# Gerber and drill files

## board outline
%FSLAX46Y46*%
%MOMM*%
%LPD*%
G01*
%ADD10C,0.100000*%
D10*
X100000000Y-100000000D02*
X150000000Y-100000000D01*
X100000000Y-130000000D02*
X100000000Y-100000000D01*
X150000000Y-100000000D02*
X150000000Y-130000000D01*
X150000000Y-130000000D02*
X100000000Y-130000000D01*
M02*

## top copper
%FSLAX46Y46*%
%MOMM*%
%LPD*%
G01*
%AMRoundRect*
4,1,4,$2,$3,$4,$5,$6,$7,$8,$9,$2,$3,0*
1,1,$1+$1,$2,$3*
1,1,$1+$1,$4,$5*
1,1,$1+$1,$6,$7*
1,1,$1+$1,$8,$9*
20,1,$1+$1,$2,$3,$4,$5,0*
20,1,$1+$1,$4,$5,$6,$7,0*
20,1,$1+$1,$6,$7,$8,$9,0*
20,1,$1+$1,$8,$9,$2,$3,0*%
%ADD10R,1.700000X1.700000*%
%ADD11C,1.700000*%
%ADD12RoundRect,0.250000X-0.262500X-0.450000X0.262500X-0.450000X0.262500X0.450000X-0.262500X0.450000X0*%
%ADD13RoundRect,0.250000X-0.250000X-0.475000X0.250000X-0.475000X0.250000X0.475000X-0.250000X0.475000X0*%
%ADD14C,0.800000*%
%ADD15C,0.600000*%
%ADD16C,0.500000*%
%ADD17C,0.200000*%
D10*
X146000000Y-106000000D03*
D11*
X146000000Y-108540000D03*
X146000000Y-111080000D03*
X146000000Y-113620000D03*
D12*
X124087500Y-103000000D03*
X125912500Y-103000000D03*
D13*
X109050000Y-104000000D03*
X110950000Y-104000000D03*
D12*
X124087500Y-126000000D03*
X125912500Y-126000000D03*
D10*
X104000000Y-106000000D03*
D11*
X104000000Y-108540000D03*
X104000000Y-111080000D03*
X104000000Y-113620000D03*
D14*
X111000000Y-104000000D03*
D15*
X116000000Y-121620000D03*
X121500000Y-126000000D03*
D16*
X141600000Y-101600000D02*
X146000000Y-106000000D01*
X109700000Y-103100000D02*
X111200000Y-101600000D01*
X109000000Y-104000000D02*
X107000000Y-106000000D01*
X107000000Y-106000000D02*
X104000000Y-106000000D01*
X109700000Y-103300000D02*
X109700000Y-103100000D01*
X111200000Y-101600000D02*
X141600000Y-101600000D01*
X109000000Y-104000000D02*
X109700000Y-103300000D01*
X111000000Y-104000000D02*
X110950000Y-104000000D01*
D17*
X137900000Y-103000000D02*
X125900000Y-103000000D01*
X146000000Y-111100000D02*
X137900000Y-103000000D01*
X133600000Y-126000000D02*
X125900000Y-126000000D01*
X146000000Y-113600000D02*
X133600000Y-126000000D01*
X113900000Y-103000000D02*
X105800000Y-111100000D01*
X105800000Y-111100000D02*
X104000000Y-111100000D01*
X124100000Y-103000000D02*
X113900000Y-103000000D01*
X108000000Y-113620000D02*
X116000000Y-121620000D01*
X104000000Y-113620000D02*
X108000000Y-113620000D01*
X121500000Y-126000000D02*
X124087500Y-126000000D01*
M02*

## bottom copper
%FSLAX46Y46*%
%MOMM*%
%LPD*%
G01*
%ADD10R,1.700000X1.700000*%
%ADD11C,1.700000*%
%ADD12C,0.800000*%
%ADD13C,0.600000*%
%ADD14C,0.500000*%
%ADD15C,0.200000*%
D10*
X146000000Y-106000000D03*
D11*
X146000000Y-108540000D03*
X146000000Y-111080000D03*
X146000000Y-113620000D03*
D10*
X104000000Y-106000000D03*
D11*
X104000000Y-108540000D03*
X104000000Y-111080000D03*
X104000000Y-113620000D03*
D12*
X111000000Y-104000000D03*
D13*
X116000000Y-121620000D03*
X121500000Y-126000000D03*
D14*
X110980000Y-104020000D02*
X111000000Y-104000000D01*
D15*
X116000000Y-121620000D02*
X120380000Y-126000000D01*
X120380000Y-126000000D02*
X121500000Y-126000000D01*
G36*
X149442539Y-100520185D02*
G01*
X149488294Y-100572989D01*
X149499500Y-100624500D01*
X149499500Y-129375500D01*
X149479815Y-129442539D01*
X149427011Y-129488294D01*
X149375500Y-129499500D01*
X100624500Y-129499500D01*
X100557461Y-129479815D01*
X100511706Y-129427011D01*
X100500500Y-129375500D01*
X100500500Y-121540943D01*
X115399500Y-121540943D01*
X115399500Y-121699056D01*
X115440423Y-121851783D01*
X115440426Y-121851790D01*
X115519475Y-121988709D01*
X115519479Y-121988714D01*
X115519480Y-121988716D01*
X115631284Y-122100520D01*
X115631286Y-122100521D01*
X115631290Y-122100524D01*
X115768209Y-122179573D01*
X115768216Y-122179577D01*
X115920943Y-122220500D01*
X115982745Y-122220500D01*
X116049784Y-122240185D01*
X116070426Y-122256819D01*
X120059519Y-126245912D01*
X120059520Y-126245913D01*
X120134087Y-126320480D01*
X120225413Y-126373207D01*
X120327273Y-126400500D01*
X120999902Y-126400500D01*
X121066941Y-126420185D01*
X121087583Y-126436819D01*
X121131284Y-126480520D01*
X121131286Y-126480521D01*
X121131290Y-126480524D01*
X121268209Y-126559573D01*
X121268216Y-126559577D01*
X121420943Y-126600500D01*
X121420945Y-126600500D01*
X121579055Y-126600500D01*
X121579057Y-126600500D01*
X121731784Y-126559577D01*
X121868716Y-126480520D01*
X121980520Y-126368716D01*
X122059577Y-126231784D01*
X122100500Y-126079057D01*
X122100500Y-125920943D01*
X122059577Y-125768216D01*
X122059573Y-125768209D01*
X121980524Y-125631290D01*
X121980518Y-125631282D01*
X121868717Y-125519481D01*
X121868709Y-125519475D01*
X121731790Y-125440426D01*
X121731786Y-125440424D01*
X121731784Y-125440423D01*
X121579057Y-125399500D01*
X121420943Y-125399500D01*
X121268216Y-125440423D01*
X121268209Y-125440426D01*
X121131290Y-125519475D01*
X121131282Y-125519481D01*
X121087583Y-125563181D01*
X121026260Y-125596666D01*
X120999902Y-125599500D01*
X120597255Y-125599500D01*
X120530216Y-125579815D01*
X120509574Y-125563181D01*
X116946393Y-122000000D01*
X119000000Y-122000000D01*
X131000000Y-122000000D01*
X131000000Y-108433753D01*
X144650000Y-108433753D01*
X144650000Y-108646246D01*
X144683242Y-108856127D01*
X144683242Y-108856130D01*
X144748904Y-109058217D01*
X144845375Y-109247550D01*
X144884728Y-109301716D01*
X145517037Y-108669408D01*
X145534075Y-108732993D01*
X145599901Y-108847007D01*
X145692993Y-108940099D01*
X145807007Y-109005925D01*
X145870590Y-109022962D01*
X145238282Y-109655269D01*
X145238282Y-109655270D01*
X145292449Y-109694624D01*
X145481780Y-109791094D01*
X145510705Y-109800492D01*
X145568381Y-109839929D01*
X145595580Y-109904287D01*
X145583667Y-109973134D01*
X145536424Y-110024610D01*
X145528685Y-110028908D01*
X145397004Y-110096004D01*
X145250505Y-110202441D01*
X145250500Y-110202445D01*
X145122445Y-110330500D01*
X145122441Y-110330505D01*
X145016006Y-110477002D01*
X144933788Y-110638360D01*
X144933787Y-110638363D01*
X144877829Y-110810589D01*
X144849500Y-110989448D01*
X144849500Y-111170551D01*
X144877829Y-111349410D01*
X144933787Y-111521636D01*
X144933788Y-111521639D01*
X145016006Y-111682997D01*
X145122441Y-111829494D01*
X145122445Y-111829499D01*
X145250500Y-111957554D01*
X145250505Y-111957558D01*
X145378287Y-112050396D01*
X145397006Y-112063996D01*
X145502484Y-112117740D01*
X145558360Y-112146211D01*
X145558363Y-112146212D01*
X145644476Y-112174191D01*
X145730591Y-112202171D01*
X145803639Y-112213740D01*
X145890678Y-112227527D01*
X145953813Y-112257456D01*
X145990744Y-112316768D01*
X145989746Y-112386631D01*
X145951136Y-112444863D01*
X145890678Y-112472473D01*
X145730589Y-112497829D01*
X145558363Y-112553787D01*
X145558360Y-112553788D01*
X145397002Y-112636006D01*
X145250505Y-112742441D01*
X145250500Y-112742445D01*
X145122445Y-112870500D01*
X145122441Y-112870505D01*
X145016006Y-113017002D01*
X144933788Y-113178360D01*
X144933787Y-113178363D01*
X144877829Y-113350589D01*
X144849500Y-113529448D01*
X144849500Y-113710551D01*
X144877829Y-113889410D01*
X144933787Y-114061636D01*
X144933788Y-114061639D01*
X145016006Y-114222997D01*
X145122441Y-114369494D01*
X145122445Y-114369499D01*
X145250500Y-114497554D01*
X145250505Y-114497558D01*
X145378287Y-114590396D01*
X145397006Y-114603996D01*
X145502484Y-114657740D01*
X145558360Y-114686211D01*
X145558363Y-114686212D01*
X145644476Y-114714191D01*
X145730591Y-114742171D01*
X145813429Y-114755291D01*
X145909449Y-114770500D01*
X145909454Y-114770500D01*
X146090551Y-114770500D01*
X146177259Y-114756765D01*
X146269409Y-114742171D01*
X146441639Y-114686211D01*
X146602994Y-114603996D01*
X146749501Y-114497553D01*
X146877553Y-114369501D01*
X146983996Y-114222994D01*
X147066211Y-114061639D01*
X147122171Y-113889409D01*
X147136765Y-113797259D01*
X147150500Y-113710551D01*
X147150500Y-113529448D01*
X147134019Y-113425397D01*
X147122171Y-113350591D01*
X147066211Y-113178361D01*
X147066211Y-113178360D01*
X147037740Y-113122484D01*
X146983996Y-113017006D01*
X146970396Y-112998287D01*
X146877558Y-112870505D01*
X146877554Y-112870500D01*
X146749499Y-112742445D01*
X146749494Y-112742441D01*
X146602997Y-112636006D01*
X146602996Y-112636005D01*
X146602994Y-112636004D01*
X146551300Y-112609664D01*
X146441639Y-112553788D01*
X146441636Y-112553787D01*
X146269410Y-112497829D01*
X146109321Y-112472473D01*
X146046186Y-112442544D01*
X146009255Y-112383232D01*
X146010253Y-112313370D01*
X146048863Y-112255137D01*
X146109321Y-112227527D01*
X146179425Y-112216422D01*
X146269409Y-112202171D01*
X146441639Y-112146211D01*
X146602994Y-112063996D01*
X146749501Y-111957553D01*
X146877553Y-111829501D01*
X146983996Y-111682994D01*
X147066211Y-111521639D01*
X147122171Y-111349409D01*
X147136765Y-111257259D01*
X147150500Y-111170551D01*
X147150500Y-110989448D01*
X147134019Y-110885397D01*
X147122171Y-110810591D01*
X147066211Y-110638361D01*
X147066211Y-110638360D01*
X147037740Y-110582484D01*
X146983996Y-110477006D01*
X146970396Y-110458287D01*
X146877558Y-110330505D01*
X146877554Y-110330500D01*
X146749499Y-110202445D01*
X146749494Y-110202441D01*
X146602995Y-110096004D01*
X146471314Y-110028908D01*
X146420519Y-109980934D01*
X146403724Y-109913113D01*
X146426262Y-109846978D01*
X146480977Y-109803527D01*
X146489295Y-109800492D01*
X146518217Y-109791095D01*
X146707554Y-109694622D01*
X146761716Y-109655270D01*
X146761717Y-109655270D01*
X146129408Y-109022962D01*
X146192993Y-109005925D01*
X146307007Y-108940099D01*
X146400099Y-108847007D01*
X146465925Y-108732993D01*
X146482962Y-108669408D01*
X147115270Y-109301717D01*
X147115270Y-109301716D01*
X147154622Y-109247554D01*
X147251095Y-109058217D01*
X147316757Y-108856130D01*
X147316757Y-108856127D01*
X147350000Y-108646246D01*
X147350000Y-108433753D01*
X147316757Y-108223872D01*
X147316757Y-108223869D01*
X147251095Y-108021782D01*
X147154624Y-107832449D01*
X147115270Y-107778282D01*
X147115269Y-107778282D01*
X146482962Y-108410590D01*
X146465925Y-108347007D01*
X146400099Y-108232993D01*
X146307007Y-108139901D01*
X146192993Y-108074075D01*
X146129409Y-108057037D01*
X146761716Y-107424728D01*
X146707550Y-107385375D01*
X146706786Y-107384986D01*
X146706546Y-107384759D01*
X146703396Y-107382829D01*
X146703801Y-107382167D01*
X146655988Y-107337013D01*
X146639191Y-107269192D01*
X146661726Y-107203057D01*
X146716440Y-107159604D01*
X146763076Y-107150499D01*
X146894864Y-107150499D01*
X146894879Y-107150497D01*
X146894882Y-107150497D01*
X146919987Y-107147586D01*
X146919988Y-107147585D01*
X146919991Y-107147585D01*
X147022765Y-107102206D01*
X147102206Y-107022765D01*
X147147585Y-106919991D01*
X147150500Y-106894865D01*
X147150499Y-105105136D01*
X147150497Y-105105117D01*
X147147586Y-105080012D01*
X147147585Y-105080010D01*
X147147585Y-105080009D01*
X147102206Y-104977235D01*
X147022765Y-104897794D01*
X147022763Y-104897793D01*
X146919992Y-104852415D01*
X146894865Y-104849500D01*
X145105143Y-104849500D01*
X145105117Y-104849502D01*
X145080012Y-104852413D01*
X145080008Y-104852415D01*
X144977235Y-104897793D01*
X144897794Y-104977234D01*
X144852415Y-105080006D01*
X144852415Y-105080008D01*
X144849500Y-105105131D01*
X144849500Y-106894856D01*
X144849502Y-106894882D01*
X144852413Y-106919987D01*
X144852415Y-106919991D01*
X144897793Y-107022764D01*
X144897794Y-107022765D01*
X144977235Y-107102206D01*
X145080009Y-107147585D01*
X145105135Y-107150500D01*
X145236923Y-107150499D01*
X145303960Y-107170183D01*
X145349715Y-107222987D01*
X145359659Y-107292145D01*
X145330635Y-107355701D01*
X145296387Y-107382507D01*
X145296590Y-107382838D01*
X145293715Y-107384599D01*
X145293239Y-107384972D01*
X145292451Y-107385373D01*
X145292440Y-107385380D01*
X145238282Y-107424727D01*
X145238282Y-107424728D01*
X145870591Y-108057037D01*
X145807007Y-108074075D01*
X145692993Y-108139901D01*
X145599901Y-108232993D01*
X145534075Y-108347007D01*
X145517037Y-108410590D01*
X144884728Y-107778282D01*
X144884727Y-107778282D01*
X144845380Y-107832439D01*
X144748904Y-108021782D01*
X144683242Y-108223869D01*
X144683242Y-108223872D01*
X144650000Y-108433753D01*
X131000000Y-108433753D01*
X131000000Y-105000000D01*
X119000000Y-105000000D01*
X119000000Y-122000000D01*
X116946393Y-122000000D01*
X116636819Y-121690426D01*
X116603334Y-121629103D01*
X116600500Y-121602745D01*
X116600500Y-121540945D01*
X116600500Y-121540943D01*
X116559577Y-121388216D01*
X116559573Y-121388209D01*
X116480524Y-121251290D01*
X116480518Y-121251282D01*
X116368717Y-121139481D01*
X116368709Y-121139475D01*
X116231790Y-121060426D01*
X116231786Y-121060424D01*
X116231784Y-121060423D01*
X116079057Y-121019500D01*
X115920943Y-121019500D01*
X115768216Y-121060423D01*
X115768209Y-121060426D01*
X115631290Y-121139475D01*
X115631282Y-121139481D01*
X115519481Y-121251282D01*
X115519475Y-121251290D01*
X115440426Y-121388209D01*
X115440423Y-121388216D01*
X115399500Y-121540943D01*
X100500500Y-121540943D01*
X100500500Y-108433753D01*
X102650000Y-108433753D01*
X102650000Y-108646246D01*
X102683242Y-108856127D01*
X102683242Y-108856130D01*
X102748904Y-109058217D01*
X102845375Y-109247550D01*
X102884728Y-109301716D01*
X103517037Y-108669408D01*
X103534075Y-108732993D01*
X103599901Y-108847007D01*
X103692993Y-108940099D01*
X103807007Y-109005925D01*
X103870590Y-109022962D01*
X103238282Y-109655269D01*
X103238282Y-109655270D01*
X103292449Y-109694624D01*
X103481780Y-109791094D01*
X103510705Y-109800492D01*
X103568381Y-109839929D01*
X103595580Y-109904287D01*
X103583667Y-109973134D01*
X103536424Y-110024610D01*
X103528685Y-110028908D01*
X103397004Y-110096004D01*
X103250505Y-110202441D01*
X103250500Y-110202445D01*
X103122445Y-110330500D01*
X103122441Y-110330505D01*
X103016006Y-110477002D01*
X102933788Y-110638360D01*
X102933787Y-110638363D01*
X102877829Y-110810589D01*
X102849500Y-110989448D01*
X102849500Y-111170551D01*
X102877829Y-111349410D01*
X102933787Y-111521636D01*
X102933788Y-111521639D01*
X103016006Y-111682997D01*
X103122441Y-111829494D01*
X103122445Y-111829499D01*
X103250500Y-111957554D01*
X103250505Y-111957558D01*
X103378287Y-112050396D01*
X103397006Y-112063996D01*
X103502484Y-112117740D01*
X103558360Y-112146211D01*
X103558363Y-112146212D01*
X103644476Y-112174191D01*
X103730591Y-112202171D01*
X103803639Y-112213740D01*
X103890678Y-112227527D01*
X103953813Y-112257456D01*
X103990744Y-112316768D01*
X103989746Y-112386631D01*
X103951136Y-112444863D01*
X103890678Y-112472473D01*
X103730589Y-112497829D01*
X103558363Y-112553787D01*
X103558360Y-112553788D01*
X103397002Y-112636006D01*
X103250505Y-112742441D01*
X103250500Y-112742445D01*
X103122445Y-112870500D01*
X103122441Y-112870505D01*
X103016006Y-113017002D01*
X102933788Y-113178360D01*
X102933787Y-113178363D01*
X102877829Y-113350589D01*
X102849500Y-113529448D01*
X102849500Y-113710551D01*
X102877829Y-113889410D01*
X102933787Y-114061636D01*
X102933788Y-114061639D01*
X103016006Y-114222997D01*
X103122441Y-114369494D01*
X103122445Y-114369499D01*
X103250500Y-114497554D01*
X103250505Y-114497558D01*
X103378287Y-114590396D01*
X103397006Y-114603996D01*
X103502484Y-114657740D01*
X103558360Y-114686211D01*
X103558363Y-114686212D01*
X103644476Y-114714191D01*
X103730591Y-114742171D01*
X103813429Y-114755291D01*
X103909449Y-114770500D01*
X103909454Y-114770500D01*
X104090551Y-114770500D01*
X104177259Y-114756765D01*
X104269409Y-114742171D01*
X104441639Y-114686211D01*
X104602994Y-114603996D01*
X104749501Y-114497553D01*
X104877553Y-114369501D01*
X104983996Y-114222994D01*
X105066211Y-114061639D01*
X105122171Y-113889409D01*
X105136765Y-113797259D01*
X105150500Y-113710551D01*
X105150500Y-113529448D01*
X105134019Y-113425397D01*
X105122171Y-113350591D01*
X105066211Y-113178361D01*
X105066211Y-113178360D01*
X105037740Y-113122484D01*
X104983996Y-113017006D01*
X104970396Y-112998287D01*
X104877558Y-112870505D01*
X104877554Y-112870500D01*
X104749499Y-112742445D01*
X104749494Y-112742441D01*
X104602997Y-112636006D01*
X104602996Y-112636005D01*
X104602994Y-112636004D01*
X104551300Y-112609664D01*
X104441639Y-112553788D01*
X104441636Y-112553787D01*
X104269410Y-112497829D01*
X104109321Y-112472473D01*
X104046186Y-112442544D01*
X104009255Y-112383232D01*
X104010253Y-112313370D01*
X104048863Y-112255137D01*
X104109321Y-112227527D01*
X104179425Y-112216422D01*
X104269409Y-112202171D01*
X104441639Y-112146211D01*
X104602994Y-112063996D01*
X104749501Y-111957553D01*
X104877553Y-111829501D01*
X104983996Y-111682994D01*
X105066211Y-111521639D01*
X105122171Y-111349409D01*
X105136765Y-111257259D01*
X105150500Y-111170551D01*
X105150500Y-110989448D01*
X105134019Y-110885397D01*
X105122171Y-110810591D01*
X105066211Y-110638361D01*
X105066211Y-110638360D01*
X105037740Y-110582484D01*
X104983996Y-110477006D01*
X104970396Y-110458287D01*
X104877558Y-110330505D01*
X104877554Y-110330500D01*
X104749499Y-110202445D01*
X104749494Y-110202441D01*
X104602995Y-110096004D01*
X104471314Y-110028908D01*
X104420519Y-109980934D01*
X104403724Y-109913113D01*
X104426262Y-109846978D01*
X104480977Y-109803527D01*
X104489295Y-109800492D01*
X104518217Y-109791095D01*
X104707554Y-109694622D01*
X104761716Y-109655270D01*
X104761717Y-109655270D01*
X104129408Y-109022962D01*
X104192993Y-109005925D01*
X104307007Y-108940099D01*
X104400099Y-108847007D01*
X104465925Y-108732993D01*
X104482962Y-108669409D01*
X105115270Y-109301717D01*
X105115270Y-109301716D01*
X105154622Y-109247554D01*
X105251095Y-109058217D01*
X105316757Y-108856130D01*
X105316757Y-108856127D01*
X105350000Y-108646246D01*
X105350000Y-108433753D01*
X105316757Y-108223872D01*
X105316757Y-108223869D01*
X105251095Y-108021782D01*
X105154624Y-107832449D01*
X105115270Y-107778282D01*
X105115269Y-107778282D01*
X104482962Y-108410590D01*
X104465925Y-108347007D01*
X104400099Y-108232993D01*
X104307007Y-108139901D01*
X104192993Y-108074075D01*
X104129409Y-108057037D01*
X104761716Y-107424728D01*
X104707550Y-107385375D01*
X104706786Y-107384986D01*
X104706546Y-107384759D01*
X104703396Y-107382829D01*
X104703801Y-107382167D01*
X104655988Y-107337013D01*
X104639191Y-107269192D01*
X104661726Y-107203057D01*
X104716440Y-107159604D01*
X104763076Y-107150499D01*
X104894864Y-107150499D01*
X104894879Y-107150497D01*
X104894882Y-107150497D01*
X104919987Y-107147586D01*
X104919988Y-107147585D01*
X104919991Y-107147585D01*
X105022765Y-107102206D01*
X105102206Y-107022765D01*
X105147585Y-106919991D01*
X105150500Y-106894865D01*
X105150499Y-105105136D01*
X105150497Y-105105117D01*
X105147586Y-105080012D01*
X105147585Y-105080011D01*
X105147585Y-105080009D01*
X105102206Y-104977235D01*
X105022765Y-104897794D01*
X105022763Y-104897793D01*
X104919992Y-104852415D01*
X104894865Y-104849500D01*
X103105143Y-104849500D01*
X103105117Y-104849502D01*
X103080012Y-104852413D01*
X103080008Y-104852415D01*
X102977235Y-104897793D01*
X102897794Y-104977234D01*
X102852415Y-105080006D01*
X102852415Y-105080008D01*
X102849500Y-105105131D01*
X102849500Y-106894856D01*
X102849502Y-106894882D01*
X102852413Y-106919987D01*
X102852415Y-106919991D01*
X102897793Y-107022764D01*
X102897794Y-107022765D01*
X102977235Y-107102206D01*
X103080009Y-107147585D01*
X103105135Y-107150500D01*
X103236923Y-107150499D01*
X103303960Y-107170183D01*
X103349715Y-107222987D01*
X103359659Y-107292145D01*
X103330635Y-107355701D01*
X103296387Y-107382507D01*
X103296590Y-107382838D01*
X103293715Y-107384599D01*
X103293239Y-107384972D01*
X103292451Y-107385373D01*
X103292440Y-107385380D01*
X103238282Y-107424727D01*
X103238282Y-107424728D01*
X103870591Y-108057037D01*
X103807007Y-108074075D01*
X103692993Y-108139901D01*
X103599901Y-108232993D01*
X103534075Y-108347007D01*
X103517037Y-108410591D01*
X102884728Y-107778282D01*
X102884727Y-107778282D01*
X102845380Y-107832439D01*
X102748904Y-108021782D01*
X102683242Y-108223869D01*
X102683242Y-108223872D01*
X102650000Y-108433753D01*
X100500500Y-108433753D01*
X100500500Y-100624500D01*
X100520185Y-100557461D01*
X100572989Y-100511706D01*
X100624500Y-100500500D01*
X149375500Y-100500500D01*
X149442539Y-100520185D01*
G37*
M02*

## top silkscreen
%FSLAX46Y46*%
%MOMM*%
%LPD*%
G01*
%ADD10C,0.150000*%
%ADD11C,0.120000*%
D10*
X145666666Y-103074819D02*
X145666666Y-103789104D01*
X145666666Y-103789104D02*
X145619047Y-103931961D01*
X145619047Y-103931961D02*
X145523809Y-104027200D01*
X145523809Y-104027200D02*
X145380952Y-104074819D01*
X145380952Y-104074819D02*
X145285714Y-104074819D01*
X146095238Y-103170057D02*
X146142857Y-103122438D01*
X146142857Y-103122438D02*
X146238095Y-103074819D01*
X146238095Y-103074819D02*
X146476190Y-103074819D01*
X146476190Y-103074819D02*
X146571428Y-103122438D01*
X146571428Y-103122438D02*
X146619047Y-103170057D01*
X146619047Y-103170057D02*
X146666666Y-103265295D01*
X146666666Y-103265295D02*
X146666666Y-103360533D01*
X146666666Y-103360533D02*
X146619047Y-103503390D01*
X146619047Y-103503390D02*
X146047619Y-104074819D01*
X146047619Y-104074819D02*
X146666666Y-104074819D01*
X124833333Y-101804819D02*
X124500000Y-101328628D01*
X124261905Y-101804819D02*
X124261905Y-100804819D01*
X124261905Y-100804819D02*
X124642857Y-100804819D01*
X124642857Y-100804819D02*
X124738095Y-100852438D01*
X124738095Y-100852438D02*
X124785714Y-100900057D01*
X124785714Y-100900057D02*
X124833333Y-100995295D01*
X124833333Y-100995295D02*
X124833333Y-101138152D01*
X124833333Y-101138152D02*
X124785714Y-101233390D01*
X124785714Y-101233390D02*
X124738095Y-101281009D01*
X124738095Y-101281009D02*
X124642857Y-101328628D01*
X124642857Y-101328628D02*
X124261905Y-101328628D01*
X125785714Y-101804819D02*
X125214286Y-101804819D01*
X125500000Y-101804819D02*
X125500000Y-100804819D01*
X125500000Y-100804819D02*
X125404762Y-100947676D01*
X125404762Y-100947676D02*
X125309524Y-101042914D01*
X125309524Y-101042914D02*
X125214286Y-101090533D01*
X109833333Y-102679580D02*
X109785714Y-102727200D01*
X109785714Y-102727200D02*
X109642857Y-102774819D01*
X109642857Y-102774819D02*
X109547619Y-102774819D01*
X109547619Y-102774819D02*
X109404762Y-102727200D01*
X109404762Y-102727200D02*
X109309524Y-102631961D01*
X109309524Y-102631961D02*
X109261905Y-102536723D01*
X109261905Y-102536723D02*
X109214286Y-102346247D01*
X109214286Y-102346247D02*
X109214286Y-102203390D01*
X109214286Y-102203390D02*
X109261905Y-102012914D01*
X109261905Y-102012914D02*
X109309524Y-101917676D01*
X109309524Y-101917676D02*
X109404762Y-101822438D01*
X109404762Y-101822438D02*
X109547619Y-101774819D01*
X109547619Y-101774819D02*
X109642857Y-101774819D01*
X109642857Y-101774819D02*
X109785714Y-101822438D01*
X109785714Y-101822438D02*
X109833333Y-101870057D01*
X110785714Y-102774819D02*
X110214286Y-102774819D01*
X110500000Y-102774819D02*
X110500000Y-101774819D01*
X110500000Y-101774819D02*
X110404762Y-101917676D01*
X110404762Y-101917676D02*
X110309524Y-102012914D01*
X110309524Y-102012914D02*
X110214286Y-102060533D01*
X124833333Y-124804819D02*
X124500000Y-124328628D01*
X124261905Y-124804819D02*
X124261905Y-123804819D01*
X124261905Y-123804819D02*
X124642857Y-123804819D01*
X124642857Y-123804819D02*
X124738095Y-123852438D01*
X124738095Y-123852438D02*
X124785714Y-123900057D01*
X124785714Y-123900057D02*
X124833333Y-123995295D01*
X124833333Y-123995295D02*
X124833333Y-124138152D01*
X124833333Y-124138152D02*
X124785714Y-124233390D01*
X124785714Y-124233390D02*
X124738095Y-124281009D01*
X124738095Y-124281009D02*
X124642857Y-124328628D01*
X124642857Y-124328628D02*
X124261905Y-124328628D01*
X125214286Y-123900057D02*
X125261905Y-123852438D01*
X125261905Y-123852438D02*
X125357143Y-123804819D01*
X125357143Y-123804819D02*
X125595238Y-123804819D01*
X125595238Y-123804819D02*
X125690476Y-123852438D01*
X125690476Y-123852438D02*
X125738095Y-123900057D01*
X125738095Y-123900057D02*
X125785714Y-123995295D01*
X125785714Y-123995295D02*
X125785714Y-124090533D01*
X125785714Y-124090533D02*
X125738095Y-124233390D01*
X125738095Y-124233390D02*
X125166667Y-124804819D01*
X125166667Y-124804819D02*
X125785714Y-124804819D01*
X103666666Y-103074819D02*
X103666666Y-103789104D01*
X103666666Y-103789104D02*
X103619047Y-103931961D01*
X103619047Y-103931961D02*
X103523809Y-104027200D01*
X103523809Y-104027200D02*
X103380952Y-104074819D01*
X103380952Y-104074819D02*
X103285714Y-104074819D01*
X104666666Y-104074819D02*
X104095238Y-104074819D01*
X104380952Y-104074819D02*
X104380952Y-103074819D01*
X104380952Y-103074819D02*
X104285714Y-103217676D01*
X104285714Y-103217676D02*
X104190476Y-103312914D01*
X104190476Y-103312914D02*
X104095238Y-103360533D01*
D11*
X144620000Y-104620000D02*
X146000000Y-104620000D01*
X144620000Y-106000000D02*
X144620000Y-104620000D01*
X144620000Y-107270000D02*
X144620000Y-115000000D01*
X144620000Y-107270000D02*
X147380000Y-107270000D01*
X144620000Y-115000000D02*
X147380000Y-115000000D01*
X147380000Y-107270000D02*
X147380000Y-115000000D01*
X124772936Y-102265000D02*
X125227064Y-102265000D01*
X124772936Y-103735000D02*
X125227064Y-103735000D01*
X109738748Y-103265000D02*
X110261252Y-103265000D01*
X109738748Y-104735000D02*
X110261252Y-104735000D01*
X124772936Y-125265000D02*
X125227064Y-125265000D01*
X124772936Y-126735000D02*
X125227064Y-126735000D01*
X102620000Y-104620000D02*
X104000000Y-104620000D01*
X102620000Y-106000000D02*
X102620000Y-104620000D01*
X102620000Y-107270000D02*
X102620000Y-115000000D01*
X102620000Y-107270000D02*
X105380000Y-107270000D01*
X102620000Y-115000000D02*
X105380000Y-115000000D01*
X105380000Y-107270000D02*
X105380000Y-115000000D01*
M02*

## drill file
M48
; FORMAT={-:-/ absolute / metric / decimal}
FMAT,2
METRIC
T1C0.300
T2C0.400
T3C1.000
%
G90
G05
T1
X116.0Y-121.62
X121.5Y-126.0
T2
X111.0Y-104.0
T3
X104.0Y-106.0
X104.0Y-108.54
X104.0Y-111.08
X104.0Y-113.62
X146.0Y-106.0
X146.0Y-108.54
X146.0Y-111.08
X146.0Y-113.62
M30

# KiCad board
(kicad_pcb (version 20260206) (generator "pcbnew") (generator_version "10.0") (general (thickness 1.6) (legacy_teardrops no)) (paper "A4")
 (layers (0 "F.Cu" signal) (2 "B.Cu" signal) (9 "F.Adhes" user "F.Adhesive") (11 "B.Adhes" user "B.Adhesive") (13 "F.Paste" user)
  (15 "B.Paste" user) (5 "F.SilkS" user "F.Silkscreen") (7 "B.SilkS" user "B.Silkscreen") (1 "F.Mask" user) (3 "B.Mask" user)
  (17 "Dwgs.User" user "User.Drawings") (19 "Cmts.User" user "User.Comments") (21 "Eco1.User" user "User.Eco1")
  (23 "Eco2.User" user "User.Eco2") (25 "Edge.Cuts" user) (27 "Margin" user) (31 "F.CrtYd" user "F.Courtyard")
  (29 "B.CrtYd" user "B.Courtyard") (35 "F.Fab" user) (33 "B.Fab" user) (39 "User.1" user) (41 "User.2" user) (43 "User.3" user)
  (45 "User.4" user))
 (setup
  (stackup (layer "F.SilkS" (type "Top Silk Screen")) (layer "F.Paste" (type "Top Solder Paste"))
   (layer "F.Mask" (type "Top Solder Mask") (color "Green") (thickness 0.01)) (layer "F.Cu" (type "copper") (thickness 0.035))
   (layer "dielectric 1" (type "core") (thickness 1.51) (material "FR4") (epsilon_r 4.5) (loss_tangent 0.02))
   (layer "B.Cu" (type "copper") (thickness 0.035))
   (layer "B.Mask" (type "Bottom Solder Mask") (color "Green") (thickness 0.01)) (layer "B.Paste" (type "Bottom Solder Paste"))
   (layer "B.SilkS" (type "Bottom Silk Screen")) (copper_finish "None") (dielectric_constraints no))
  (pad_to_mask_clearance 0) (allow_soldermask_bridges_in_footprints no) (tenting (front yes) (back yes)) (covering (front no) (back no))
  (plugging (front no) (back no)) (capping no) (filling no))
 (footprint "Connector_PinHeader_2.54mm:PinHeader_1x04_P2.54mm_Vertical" (layer "F.Cu") (at 146 106)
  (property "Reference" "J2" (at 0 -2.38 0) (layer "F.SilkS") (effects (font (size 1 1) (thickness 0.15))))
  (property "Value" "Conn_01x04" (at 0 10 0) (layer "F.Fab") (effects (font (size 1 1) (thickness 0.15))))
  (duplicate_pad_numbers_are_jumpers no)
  (fp_line (start -1.38 -1.38) (end 0 -1.38) (stroke (width 0.12) (type solid)) (layer "F.SilkS"))
  (fp_line (start -1.38 0) (end -1.38 -1.38) (stroke (width 0.12) (type solid)) (layer "F.SilkS"))
  (fp_line (start -1.38 1.27) (end -1.38 9) (stroke (width 0.12) (type solid)) (layer "F.SilkS"))
  (fp_line (start -1.38 1.27) (end 1.38 1.27) (stroke (width 0.12) (type solid)) (layer "F.SilkS"))
  (fp_line (start -1.38 9) (end 1.38 9) (stroke (width 0.12) (type solid)) (layer "F.SilkS"))
  (fp_line (start 1.38 1.27) (end 1.38 9) (stroke (width 0.12) (type solid)) (layer "F.SilkS"))
  (pad "1" thru_hole rect (at 0 0) (size 1.7 1.7) (drill 1) (layers "*.Cu" "*.Mask") (remove_unused_layers no) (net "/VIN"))
  (pad "2" thru_hole circle (at 0 2.54) (size 1.7 1.7) (drill 1) (layers "*.Cu" "*.Mask") (remove_unused_layers no) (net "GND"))
  (pad "3" thru_hole circle (at 0 5.08) (size 1.7 1.7) (drill 1) (layers "*.Cu" "*.Mask") (remove_unused_layers no) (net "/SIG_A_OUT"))
  (pad "4" thru_hole circle (at 0 7.62) (size 1.7 1.7) (drill 1) (layers "*.Cu" "*.Mask") (remove_unused_layers no) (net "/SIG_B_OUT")))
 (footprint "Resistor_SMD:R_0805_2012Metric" (layer "F.Cu") (at 125 103)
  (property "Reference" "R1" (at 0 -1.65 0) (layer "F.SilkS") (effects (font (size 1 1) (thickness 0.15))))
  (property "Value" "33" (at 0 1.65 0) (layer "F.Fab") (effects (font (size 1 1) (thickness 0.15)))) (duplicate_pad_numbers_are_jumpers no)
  (fp_line (start -0.227064 -0.735) (end 0.227064 -0.735) (stroke (width 0.12) (type solid)) (layer "F.SilkS"))
  (fp_line (start -0.227064 0.735) (end 0.227064 0.735) (stroke (width 0.12) (type solid)) (layer "F.SilkS"))
  (pad "1" smd roundrect (at -0.9125 0) (size 1.025 1.4) (layers "F.Cu" "F.Mask" "F.Paste") (roundrect_rratio 0.243902) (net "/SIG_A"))
  (pad "2" smd roundrect (at 0.9125 0) (size 1.025 1.4) (layers "F.Cu" "F.Mask" "F.Paste") (roundrect_rratio 0.243902) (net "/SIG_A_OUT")))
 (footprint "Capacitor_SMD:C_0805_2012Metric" (layer "F.Cu") (at 110 104)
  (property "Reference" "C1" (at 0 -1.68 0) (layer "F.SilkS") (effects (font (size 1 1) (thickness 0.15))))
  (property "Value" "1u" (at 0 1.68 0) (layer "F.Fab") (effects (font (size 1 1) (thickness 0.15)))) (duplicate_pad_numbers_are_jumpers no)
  (fp_line (start -0.261252 -0.735) (end 0.261252 -0.735) (stroke (width 0.12) (type solid)) (layer "F.SilkS"))
  (fp_line (start -0.261252 0.735) (end 0.261252 0.735) (stroke (width 0.12) (type solid)) (layer "F.SilkS"))
  (pad "1" smd roundrect (at -0.95 0) (size 1 1.45) (layers "F.Cu" "F.Mask" "F.Paste") (roundrect_rratio 0.25) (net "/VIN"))
  (pad "2" smd roundrect (at 0.95 0) (size 1 1.45) (layers "F.Cu" "F.Mask" "F.Paste") (roundrect_rratio 0.25) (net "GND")))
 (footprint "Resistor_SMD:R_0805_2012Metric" (layer "F.Cu") (at 125 126)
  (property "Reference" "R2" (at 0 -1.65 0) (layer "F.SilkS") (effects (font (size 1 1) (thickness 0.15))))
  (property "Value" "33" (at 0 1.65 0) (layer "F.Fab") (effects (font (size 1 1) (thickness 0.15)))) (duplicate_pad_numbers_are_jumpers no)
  (fp_line (start -0.227064 -0.735) (end 0.227064 -0.735) (stroke (width 0.12) (type solid)) (layer "F.SilkS"))
  (fp_line (start -0.227064 0.735) (end 0.227064 0.735) (stroke (width 0.12) (type solid)) (layer "F.SilkS"))
  (pad "1" smd roundrect (at -0.9125 0) (size 1.025 1.4) (layers "F.Cu" "F.Mask" "F.Paste") (roundrect_rratio 0.243902) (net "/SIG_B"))
  (pad "2" smd roundrect (at 0.9125 0) (size 1.025 1.4) (layers "F.Cu" "F.Mask" "F.Paste") (roundrect_rratio 0.243902) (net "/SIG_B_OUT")))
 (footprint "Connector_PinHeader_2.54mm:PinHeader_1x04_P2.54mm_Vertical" (layer "F.Cu") (at 104 106)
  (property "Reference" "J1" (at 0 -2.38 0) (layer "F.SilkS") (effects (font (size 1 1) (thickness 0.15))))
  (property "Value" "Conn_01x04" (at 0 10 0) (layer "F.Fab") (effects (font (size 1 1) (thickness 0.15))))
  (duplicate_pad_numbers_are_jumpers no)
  (fp_line (start -1.38 -1.38) (end 0 -1.38) (stroke (width 0.12) (type solid)) (layer "F.SilkS"))
  (fp_line (start -1.38 0) (end -1.38 -1.38) (stroke (width 0.12) (type solid)) (layer "F.SilkS"))
  (fp_line (start -1.38 1.27) (end -1.38 9) (stroke (width 0.12) (type solid)) (layer "F.SilkS"))
  (fp_line (start -1.38 1.27) (end 1.38 1.27) (stroke (width 0.12) (type solid)) (layer "F.SilkS"))
  (fp_line (start -1.38 9) (end 1.38 9) (stroke (width 0.12) (type solid)) (layer "F.SilkS"))
  (fp_line (start 1.38 1.27) (end 1.38 9) (stroke (width 0.12) (type solid)) (layer "F.SilkS"))
  (pad "1" thru_hole rect (at 0 0) (size 1.7 1.7) (drill 1) (layers "*.Cu" "*.Mask") (remove_unused_layers no) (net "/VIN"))
  (pad "2" thru_hole circle (at 0 2.54) (size 1.7 1.7) (drill 1) (layers "*.Cu" "*.Mask") (remove_unused_layers no) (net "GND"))
  (pad "3" thru_hole circle (at 0 5.08) (size 1.7 1.7) (drill 1) (layers "*.Cu" "*.Mask") (remove_unused_layers no) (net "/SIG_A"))
  (pad "4" thru_hole circle (at 0 7.62) (size 1.7 1.7) (drill 1) (layers "*.Cu" "*.Mask") (remove_unused_layers no) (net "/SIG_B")))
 (gr_line (start 100 100) (end 150 100) (stroke (width 0.1) (type default)) (layer "Edge.Cuts"))
 (gr_line (start 100 130) (end 100 100) (stroke (width 0.1) (type default)) (layer "Edge.Cuts"))
 (gr_line (start 150 100) (end 150 130) (stroke (width 0.1) (type default)) (layer "Edge.Cuts"))
 (gr_line (start 150 130) (end 100 130) (stroke (width 0.1) (type default)) (layer "Edge.Cuts"))
 (segment (start 141.6 101.6) (end 146 106) (width 0.5) (layer "F.Cu") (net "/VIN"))
 (segment (start 109.7 103.1) (end 111.2 101.6) (width 0.5) (layer "F.Cu") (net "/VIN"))
 (segment (start 109 104) (end 107 106) (width 0.5) (layer "F.Cu") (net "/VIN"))
 (segment (start 107 106) (end 104 106) (width 0.5) (layer "F.Cu") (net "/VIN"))
 (segment (start 109.7 103.3) (end 109.7 103.1) (width 0.5) (layer "F.Cu") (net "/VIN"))
 (segment (start 111.2 101.6) (end 141.6 101.6) (width 0.5) (layer "F.Cu") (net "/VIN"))
 (segment (start 109 104) (end 109.7 103.3) (width 0.5) (layer "F.Cu") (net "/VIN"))
 (segment (start 111 104) (end 110.95 104) (width 0.5) (layer "F.Cu") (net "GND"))
 (via (at 111 104) (size 0.8) (drill 0.4) (layers "F.Cu" "B.Cu") (capping yes) (filling yes) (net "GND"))
 (segment (start 110.98 104.02) (end 111 104) (width 0.5) (layer "B.Cu") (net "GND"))
 (segment (start 137.9 103) (end 125.9 103) (width 0.2) (layer "F.Cu") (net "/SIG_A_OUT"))
 (segment (start 146 111.1) (end 137.9 103) (width 0.2) (layer "F.Cu") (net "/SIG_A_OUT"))
 (segment (start 133.6 126) (end 125.9 126) (width 0.2) (layer "F.Cu") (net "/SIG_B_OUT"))
 (segment (start 146 113.6) (end 133.6 126) (width 0.2) (layer "F.Cu") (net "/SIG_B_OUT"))
 (segment (start 113.9 103) (end 105.8 111.1) (width 0.2) (layer "F.Cu") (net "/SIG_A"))
 (segment (start 105.8 111.1) (end 104 111.1) (width 0.2) (layer "F.Cu") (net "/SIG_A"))
 (segment (start 124.1 103) (end 113.9 103) (width 0.2) (layer "F.Cu") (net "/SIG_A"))
 (segment (start 108 113.62) (end 116 121.62) (width 0.2) (locked yes) (layer "F.Cu") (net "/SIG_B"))
 (segment (start 104 113.62) (end 108 113.62) (width 0.2) (locked yes) (layer "F.Cu") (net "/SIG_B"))
 (segment (start 121.5 126) (end 124.0875 126) (width 0.2) (locked yes) (layer "F.Cu") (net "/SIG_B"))
 (via (at 116 121.62) (size 0.6) (drill 0.3) (layers "F.Cu" "B.Cu") (locked yes) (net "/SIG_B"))
 (via (at 121.5 126) (size 0.6) (drill 0.3) (layers "F.Cu" "B.Cu") (locked yes) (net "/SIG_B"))
 (segment (start 116 121.62) (end 120.38 126) (width 0.2) (locked yes) (layer "B.Cu") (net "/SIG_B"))
 (segment (start 120.38 126) (end 121.5 126) (width 0.2) (locked yes) (layer "B.Cu") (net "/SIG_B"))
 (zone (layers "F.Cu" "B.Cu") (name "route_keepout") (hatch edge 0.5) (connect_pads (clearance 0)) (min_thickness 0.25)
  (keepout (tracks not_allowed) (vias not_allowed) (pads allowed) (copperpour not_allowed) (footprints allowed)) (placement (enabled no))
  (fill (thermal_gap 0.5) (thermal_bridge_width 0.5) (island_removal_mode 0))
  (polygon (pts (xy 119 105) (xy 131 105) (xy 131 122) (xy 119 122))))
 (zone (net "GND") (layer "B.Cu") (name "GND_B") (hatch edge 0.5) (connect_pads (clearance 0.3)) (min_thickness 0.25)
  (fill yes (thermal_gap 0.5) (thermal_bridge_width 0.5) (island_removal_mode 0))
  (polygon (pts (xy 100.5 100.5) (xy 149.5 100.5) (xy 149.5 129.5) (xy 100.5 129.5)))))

